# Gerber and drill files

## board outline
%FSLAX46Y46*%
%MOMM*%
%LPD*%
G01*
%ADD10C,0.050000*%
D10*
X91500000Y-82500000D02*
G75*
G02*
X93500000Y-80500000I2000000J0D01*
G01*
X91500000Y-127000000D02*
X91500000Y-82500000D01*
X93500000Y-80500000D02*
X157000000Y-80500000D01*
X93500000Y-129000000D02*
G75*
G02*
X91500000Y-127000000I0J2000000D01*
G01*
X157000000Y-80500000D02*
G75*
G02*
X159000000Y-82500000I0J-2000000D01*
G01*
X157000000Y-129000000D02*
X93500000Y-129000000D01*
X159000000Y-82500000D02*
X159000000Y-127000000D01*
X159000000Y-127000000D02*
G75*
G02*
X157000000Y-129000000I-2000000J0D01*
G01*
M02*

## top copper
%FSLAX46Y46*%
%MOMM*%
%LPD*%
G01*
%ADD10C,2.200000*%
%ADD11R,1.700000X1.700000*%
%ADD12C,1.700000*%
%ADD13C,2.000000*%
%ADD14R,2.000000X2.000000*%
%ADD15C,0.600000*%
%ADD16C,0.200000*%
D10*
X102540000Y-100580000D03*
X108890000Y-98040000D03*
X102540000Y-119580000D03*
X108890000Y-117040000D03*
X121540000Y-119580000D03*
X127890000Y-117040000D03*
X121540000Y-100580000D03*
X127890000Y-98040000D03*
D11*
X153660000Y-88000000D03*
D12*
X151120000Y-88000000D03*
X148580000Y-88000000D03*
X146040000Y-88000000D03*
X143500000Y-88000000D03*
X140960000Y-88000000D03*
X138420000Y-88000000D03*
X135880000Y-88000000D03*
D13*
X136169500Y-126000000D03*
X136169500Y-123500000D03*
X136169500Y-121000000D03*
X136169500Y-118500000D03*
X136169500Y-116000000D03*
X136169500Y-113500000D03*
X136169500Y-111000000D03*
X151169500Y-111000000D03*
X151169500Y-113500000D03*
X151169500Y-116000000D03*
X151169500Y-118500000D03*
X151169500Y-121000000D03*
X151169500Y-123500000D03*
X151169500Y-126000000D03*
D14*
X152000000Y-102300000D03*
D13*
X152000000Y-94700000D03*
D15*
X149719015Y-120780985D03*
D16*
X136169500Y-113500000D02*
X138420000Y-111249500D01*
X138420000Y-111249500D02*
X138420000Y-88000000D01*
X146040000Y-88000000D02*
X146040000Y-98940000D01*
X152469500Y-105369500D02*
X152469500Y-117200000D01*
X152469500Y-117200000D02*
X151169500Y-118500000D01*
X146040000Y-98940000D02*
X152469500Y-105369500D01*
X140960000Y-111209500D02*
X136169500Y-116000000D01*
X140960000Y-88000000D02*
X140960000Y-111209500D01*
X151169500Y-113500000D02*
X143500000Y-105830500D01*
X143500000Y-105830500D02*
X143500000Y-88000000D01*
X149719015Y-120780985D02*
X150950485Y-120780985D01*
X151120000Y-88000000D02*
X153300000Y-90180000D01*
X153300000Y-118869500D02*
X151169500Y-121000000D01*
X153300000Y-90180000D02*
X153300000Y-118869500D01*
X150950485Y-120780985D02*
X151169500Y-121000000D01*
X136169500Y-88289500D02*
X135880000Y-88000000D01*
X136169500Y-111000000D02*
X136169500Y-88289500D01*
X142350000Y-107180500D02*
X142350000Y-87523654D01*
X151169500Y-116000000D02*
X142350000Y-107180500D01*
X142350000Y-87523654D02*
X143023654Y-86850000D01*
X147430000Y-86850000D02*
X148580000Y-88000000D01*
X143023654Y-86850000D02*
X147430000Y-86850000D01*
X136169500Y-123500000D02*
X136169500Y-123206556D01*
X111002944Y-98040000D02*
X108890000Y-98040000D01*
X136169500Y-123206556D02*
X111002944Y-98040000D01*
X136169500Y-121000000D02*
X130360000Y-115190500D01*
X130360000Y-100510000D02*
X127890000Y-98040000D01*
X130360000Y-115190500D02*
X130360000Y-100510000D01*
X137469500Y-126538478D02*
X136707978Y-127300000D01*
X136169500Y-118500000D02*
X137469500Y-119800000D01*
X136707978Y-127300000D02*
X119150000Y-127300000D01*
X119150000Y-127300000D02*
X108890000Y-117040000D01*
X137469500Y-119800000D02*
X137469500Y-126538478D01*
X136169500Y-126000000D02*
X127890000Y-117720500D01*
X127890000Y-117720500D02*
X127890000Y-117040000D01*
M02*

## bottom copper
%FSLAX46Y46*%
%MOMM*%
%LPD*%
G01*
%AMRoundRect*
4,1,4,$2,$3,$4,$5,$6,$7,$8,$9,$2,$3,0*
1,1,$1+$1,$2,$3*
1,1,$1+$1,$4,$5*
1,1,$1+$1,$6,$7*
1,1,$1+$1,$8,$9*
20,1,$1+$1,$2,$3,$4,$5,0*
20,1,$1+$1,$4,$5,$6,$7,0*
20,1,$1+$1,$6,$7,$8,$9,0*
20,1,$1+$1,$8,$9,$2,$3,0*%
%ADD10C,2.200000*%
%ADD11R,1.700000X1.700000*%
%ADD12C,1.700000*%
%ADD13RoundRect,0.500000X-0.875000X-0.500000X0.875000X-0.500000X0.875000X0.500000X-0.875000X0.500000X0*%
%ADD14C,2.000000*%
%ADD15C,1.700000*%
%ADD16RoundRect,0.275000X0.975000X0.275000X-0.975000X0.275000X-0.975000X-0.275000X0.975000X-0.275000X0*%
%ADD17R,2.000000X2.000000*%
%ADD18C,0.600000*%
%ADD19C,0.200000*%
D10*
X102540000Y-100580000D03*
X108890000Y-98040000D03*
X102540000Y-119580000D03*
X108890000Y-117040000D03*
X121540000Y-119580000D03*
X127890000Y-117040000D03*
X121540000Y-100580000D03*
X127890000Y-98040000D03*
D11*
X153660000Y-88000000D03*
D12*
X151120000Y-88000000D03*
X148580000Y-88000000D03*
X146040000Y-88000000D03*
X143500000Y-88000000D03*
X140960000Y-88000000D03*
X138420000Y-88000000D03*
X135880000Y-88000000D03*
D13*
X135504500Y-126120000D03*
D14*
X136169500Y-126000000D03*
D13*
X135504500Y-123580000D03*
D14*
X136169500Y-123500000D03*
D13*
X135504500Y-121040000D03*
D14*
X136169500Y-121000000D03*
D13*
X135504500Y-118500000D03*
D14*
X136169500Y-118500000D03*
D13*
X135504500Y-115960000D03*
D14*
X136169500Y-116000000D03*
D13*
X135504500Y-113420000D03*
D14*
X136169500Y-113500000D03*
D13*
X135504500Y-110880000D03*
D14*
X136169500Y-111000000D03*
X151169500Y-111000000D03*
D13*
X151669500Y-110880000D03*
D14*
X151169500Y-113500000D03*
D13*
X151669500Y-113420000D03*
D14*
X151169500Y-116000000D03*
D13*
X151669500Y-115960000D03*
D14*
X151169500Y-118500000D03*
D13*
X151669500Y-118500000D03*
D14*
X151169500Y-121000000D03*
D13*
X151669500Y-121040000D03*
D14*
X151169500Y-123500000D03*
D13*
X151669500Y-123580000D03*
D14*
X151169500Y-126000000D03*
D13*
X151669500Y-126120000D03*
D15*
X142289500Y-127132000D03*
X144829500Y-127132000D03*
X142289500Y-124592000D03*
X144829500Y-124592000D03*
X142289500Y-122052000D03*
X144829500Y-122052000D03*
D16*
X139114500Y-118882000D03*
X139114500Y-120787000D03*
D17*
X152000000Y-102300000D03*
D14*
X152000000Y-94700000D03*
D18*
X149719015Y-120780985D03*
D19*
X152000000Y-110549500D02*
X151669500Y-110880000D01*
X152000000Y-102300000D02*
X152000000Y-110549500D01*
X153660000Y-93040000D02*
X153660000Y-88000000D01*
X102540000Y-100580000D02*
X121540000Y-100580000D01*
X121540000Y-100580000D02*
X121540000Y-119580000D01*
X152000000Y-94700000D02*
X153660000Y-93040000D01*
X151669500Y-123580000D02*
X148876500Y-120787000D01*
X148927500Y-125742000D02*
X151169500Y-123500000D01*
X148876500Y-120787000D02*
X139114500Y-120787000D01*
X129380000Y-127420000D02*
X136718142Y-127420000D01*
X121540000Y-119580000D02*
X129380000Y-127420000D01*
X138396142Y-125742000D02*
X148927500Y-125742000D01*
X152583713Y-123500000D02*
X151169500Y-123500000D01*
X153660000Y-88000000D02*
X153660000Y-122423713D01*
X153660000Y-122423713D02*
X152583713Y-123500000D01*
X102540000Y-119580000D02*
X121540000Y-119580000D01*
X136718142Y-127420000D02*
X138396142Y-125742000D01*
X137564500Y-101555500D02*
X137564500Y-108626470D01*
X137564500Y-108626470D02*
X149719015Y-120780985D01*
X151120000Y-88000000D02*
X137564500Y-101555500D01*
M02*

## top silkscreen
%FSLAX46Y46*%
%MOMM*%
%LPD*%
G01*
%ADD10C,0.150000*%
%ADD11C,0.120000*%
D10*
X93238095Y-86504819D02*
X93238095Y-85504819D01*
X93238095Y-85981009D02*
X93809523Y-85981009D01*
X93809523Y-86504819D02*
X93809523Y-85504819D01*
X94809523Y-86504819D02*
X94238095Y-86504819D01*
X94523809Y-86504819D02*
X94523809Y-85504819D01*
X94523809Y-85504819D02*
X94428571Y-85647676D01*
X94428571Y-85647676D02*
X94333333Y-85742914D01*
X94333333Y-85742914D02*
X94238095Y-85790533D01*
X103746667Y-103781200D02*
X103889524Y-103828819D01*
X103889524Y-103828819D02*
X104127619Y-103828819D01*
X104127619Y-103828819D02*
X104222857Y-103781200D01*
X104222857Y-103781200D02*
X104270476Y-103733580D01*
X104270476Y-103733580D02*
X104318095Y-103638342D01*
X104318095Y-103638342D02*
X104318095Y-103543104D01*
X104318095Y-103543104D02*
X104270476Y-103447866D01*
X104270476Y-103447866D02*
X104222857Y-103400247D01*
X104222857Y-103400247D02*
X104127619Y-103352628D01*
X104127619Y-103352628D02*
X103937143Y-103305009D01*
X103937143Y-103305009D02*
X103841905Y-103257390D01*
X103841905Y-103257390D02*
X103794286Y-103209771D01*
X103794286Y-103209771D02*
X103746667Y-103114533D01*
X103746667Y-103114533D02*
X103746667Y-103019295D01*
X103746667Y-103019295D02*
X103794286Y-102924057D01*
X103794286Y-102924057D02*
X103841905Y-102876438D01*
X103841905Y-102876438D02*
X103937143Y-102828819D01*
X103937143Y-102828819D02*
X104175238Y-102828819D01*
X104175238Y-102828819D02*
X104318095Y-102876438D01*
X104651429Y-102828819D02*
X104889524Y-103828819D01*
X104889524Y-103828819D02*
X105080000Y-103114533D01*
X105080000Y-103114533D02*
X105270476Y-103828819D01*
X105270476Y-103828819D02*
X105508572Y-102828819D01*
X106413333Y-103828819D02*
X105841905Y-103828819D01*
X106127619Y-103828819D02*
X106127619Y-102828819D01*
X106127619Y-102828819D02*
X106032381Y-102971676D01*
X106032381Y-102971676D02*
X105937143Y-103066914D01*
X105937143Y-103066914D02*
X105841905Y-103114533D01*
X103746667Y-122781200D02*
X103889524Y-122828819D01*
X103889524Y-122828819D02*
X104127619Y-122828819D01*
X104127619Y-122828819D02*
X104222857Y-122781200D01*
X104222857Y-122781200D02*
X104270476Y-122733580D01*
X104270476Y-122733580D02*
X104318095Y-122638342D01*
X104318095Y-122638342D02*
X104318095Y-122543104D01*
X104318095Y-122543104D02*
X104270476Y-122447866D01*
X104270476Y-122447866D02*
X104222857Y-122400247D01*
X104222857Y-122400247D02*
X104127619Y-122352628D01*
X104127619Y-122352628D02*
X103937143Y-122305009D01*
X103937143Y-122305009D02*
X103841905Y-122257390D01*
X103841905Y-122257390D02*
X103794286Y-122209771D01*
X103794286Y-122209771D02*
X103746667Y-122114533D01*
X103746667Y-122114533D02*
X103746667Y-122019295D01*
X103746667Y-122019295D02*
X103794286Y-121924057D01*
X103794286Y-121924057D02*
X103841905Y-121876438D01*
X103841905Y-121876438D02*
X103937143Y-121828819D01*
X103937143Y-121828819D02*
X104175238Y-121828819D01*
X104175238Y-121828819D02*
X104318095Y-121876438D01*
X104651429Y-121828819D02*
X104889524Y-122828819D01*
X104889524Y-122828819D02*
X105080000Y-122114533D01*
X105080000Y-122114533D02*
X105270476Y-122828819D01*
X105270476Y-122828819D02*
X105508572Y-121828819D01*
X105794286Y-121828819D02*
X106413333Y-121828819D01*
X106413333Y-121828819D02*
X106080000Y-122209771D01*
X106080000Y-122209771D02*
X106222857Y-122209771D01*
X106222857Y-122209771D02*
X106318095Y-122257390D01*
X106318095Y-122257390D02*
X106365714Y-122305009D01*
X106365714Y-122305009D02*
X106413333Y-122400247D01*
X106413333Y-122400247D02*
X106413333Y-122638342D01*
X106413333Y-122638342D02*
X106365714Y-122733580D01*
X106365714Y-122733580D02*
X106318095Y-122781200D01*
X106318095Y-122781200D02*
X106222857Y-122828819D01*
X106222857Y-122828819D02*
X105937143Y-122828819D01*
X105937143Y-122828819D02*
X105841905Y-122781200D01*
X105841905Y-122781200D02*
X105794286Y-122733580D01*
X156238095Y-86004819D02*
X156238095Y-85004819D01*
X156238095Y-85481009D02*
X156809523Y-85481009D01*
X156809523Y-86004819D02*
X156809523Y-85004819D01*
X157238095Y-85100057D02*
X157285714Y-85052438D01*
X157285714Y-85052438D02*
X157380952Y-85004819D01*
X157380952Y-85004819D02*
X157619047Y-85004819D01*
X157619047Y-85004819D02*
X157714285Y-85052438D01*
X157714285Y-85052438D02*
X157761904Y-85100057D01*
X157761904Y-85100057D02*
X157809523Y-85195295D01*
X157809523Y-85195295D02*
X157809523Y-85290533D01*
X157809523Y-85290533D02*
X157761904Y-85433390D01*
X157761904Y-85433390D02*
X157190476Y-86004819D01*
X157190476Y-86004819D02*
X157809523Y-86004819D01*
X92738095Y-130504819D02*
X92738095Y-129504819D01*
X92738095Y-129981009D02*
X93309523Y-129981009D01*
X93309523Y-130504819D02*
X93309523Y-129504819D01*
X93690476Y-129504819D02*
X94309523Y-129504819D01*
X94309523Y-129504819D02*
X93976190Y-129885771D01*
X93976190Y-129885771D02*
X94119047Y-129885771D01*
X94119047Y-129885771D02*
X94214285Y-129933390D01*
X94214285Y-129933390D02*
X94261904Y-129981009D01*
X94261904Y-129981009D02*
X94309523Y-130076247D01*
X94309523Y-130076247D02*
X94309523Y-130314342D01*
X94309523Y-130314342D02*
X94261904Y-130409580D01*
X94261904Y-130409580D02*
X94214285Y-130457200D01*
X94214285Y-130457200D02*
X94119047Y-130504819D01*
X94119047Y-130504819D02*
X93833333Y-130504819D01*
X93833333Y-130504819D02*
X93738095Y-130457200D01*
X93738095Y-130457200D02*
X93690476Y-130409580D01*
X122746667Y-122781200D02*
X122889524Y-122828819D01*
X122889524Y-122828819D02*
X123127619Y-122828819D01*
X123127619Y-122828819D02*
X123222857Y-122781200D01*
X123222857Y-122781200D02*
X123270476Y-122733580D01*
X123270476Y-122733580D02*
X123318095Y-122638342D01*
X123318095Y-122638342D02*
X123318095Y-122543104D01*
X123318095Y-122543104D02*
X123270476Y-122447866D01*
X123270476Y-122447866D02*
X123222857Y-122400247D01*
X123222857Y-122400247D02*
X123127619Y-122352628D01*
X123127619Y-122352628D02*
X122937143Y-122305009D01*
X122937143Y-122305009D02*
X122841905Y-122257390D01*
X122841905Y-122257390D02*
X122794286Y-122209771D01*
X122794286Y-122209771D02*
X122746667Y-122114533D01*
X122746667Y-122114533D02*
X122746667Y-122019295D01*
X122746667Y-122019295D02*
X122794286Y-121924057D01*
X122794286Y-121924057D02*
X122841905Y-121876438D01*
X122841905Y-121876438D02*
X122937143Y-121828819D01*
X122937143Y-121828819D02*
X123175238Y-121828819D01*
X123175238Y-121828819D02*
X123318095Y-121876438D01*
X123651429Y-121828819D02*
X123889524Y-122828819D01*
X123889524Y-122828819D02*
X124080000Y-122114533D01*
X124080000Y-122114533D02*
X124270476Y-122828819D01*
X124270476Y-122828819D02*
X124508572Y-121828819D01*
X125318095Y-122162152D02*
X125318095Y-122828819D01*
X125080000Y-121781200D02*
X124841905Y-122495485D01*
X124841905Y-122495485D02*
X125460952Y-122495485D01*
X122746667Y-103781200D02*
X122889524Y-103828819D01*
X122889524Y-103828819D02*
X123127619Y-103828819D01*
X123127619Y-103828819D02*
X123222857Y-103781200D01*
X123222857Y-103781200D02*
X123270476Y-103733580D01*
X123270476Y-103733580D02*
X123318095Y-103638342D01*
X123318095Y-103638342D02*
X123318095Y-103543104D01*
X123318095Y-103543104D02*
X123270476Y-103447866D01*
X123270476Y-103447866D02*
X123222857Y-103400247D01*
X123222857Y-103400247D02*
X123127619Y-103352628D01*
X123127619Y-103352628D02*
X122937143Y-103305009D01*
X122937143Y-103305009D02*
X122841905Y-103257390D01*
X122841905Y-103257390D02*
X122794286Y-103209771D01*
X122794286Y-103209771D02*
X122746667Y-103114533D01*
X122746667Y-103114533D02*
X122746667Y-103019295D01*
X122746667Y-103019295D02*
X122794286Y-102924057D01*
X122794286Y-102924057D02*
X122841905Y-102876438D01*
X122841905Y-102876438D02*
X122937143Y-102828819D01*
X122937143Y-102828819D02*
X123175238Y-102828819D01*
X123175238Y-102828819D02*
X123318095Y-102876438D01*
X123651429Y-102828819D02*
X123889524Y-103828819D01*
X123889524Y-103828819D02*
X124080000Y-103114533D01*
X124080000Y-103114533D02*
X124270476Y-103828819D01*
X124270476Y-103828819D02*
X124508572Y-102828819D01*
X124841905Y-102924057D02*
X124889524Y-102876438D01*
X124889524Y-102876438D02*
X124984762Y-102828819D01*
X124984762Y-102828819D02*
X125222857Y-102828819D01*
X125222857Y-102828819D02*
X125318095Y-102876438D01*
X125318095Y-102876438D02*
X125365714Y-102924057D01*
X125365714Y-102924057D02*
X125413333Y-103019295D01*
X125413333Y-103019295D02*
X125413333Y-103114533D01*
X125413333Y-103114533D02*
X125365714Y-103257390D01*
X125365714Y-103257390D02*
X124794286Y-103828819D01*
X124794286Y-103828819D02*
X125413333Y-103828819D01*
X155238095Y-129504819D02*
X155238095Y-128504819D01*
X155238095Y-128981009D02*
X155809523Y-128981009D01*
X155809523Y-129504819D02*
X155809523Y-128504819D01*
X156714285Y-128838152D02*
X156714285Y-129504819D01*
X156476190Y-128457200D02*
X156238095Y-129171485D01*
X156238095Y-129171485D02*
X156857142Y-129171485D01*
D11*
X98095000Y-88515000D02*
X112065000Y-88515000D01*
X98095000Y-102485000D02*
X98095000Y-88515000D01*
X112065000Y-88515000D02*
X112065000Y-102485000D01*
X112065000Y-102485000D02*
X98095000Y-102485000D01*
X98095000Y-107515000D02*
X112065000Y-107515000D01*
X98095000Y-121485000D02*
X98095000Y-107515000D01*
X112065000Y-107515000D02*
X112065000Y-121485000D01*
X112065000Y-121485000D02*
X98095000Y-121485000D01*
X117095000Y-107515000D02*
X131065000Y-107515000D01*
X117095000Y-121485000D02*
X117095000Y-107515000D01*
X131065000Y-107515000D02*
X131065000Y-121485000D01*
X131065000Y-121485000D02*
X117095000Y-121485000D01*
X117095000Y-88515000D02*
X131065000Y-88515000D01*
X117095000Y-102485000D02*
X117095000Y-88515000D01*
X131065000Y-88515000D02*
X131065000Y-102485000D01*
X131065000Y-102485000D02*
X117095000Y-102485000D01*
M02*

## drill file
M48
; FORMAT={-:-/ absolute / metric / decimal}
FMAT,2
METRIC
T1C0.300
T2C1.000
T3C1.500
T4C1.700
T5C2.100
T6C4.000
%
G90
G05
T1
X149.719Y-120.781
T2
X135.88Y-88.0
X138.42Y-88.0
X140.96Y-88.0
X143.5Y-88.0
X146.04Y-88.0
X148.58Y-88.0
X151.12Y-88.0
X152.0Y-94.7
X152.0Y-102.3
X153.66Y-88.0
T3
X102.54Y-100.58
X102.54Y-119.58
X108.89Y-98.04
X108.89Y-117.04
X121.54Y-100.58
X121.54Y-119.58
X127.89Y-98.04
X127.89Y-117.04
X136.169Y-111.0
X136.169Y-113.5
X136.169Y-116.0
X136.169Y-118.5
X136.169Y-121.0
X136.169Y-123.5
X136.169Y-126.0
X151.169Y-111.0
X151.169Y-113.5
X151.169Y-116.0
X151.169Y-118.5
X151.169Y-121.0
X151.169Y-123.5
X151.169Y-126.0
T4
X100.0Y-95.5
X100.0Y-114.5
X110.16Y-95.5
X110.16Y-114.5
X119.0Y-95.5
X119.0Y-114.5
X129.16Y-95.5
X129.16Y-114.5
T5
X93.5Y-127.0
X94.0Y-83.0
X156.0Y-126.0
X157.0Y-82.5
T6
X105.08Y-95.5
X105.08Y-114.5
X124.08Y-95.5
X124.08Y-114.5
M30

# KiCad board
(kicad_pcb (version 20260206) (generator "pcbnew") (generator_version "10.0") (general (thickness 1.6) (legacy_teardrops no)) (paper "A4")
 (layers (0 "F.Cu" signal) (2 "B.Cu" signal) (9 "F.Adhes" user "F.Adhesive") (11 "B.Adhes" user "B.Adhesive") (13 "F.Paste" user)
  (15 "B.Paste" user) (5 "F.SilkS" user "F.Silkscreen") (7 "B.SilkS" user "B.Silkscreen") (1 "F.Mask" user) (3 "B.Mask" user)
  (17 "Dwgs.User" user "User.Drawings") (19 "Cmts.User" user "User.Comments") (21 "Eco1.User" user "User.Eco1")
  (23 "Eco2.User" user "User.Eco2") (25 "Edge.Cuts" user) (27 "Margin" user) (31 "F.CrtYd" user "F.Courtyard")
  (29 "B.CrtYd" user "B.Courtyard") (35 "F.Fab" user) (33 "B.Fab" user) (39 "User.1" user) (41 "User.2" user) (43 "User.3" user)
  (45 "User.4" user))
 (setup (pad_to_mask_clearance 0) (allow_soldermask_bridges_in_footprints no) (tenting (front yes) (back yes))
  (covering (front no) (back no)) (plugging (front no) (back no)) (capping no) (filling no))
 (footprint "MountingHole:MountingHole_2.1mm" (layer "F.Cu") (at 94 83 180)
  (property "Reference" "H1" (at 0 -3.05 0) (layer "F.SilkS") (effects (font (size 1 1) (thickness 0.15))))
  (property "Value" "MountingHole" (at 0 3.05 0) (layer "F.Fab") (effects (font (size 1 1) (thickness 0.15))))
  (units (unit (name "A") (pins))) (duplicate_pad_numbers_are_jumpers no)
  (pad "" np_thru_hole circle (at 0 0 180) (size 2.1 2.1) (drill 2.1) (layers "*.Cu" "*.Mask")))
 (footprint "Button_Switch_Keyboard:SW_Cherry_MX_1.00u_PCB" (layer "F.Cu") (at 102.54 100.58 180)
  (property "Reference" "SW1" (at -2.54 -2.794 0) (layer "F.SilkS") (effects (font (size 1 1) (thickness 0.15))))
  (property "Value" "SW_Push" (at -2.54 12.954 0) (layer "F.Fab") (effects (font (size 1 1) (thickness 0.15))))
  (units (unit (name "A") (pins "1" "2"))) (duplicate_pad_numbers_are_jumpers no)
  (fp_line (start 4.445 12.065) (end -9.525 12.065) (stroke (width 0.12) (type solid)) (layer "F.SilkS"))
  (fp_line (start 4.445 -1.905) (end 4.445 12.065) (stroke (width 0.12) (type solid)) (layer "F.SilkS"))
  (fp_line (start -9.525 12.065) (end -9.525 -1.905) (stroke (width 0.12) (type solid)) (layer "F.SilkS"))
  (fp_line (start -9.525 -1.905) (end 4.445 -1.905) (stroke (width 0.12) (type solid)) (layer "F.SilkS"))
  (pad "" np_thru_hole circle (at -7.62 5.08 180) (size 1.7 1.7) (drill 1.7) (layers "*.Cu" "*.Mask"))
  (pad "" np_thru_hole circle (at -2.54 5.08 180) (size 4 4) (drill 4) (layers "*.Cu" "*.Mask"))
  (pad "" np_thru_hole circle (at 2.54 5.08 180) (size 1.7 1.7) (drill 1.7) (layers "*.Cu" "*.Mask"))
  (pad "1" thru_hole circle (at 0 0 180) (size 2.2 2.2) (drill 1.5) (layers "*.Cu" "*.Mask") (remove_unused_layers no) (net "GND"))
  (pad "2" thru_hole circle (at -6.35 2.54 180) (size 2.2 2.2) (drill 1.5) (layers "*.Cu" "*.Mask") (remove_unused_layers no)
   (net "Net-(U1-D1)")))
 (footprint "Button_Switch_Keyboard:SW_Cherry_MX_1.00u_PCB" (layer "F.Cu") (at 102.54 119.58 180)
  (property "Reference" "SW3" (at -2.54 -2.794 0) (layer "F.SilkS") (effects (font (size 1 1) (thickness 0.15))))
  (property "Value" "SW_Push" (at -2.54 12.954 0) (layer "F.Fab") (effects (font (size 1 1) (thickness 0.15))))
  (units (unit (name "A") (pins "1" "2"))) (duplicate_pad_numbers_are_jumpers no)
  (fp_line (start 4.445 12.065) (end -9.525 12.065) (stroke (width 0.12) (type solid)) (layer "F.SilkS"))
  (fp_line (start 4.445 -1.905) (end 4.445 12.065) (stroke (width 0.12) (type solid)) (layer "F.SilkS"))
  (fp_line (start -9.525 12.065) (end -9.525 -1.905) (stroke (width 0.12) (type solid)) (layer "F.SilkS"))
  (fp_line (start -9.525 -1.905) (end 4.445 -1.905) (stroke (width 0.12) (type solid)) (layer "F.SilkS"))
  (pad "" np_thru_hole circle (at -7.62 5.08 180) (size 1.7 1.7) (drill 1.7) (layers "*.Cu" "*.Mask"))
  (pad "" np_thru_hole circle (at -2.54 5.08 180) (size 4 4) (drill 4) (layers "*.Cu" "*.Mask"))
  (pad "" np_thru_hole circle (at 2.54 5.08 180) (size 1.7 1.7) (drill 1.7) (layers "*.Cu" "*.Mask"))
  (pad "1" thru_hole circle (at 0 0 180) (size 2.2 2.2) (drill 1.5) (layers "*.Cu" "*.Mask") (remove_unused_layers no) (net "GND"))
  (pad "2" thru_hole circle (at -6.35 2.54 180) (size 2.2 2.2) (drill 1.5) (layers "*.Cu" "*.Mask") (remove_unused_layers no)
   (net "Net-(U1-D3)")))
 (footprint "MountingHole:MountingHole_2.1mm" (layer "F.Cu") (at 157 82.5 180)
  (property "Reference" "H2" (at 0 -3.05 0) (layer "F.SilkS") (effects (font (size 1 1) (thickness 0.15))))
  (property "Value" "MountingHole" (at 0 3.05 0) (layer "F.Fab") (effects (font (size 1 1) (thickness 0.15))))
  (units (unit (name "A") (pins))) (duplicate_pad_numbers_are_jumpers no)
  (pad "" np_thru_hole circle (at 0 0 180) (size 2.1 2.1) (drill 2.1) (layers "*.Cu" "*.Mask")))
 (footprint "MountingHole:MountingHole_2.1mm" (layer "F.Cu") (at 93.5 127 180)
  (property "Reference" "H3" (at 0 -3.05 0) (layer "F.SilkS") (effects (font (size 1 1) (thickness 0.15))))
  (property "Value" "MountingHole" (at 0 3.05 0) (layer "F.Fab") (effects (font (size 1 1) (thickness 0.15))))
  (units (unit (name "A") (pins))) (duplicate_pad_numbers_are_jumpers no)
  (pad "" np_thru_hole circle (at 0 0 180) (size 2.1 2.1) (drill 2.1) (layers "*.Cu" "*.Mask")))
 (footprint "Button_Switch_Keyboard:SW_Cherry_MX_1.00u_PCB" (layer "F.Cu") (at 121.54 119.58 180)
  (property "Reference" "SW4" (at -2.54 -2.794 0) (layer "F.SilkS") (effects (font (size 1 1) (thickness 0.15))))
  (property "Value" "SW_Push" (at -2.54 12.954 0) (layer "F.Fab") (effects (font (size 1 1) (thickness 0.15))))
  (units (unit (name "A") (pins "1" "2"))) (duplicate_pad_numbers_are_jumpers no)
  (fp_line (start 4.445 12.065) (end -9.525 12.065) (stroke (width 0.12) (type solid)) (layer "F.SilkS"))
  (fp_line (start 4.445 -1.905) (end 4.445 12.065) (stroke (width 0.12) (type solid)) (layer "F.SilkS"))
  (fp_line (start -9.525 12.065) (end -9.525 -1.905) (stroke (width 0.12) (type solid)) (layer "F.SilkS"))
  (fp_line (start -9.525 -1.905) (end 4.445 -1.905) (stroke (width 0.12) (type solid)) (layer "F.SilkS"))
  (pad "" np_thru_hole circle (at -7.62 5.08 180) (size 1.7 1.7) (drill 1.7) (layers "*.Cu" "*.Mask"))
  (pad "" np_thru_hole circle (at -2.54 5.08 180) (size 4 4) (drill 4) (layers "*.Cu" "*.Mask"))
  (pad "" np_thru_hole circle (at 2.54 5.08 180) (size 1.7 1.7) (drill 1.7) (layers "*.Cu" "*.Mask"))
  (pad "1" thru_hole circle (at 0 0 180) (size 2.2 2.2) (drill 1.5) (layers "*.Cu" "*.Mask") (remove_unused_layers no) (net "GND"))
  (pad "2" thru_hole circle (at -6.35 2.54 180) (size 2.2 2.2) (drill 1.5) (layers "*.Cu" "*.Mask") (remove_unused_layers no)
   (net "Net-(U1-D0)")))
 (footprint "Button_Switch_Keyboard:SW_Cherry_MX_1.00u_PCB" (layer "F.Cu") (at 121.54 100.58 180)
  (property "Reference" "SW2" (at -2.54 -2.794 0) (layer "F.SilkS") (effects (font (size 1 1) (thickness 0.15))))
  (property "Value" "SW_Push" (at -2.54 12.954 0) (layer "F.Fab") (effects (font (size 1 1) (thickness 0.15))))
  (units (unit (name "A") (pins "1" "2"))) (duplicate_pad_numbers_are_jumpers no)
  (fp_line (start 4.445 12.065) (end -9.525 12.065) (stroke (width 0.12) (type solid)) (layer "F.SilkS"))
  (fp_line (start 4.445 -1.905) (end 4.445 12.065) (stroke (width 0.12) (type solid)) (layer "F.SilkS"))
  (fp_line (start -9.525 12.065) (end -9.525 -1.905) (stroke (width 0.12) (type solid)) (layer "F.SilkS"))
  (fp_line (start -9.525 -1.905) (end 4.445 -1.905) (stroke (width 0.12) (type solid)) (layer "F.SilkS"))
  (pad "" np_thru_hole circle (at -7.62 5.08 180) (size 1.7 1.7) (drill 1.7) (layers "*.Cu" "*.Mask"))
  (pad "" np_thru_hole circle (at -2.54 5.08 180) (size 4 4) (drill 4) (layers "*.Cu" "*.Mask"))
  (pad "" np_thru_hole circle (at 2.54 5.08 180) (size 1.7 1.7) (drill 1.7) (layers "*.Cu" "*.Mask"))
  (pad "1" thru_hole circle (at 0 0 180) (size 2.2 2.2) (drill 1.5) (layers "*.Cu" "*.Mask") (remove_unused_layers no) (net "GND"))
  (pad "2" thru_hole circle (at -6.35 2.54 180) (size 2.2 2.2) (drill 1.5) (layers "*.Cu" "*.Mask") (remove_unused_layers no)
   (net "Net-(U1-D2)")))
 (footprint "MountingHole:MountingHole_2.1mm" (layer "F.Cu") (at 156 126 180)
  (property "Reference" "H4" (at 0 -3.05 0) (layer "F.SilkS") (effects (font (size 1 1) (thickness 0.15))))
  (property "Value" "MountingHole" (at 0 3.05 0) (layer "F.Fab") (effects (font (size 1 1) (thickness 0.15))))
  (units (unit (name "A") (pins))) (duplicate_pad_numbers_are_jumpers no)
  (pad "" np_thru_hole circle (at 0 0 180) (size 2.1 2.1) (drill 2.1) (layers "*.Cu" "*.Mask")))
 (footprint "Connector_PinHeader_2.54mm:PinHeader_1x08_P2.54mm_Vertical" (layer "B.Cu") (at 153.66 88 90)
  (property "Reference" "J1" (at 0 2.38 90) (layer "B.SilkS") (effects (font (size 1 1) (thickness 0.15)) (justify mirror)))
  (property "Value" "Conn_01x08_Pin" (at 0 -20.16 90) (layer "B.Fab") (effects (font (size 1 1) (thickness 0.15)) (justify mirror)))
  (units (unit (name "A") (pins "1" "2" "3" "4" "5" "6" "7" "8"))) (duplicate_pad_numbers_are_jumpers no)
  (pad "1" thru_hole rect (at 0 0 90) (size 1.7 1.7) (drill 1) (layers "*.Cu" "*.Mask") (remove_unused_layers no) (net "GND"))
  (pad "2" thru_hole circle (at 0 -2.54 90) (size 1.7 1.7) (drill 1) (layers "*.Cu" "*.Mask") (remove_unused_layers no) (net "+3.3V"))
  (pad "3" thru_hole circle (at 0 -5.08 90) (size 1.7 1.7) (drill 1) (layers "*.Cu" "*.Mask") (remove_unused_layers no) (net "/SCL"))
  (pad "4" thru_hole circle (at 0 -7.62 90) (size 1.7 1.7) (drill 1) (layers "*.Cu" "*.Mask") (remove_unused_layers no) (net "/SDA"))
  (pad "5" thru_hole circle (at 0 -10.16 90) (size 1.7 1.7) (drill 1) (layers "*.Cu" "*.Mask") (remove_unused_layers no) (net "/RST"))
  (pad "6" thru_hole circle (at 0 -12.7 90) (size 1.7 1.7) (drill 1) (layers "*.Cu" "*.Mask") (remove_unused_layers no) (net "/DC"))
  (pad "7" thru_hole circle (at 0 -15.24 90) (size 1.7 1.7) (drill 1) (layers "*.Cu" "*.Mask") (remove_unused_layers no) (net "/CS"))
  (pad "8" thru_hole circle (at 0 -17.78 90) (size 1.7 1.7) (drill 1) (layers "*.Cu" "*.Mask") (remove_unused_layers no) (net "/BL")))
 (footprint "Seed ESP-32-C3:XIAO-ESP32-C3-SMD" (layer "B.Cu") (at 134.6695 108)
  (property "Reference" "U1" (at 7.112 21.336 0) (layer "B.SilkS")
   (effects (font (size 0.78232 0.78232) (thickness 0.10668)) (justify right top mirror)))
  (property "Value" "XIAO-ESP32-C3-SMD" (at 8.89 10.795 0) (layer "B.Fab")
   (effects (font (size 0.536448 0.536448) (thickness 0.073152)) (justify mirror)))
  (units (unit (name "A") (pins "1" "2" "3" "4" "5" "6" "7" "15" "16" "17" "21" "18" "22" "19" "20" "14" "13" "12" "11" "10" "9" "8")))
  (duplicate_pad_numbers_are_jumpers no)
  (pad "1" smd roundrect (at 0.835 18.12) (size 2.75 2) (layers "B.Cu" "B.Mask" "B.Paste") (roundrect_rratio 0.25) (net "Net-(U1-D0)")
   (solder_mask_margin 0.0508) (thermal_bridge_angle 45))
  (pad "1" thru_hole circle (at 1.5 18) (size 2 2) (drill 1.5) (layers "*.Cu" "*.Mask") (remove_unused_layers no) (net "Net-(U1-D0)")
   (thermal_bridge_angle 90))
  (pad "2" smd roundrect (at 0.835 15.58) (size 2.75 2) (layers "B.Cu" "B.Mask" "B.Paste") (roundrect_rratio 0.25) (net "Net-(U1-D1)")
   (solder_mask_margin 0.0508) (thermal_bridge_angle 45))
  (pad "2" thru_hole circle (at 1.5 15.5) (size 2 2) (drill 1.5) (layers "*.Cu" "*.Mask") (remove_unused_layers no) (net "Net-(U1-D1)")
   (thermal_bridge_angle 90))
  (pad "3" smd roundrect (at 0.835 13.04) (size 2.75 2) (layers "B.Cu" "B.Mask" "B.Paste") (roundrect_rratio 0.25) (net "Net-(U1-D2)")
   (solder_mask_margin 0.0508) (thermal_bridge_angle 45))
  (pad "3" thru_hole circle (at 1.5 13) (size 2 2) (drill 1.5) (layers "*.Cu" "*.Mask") (remove_unused_layers no) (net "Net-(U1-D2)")
   (thermal_bridge_angle 90))
  (pad "4" smd roundrect (at 0.835 10.5) (size 2.75 2) (layers "B.Cu" "B.Mask" "B.Paste") (roundrect_rratio 0.25) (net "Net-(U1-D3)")
   (solder_mask_margin 0.0508) (thermal_bridge_angle 45))
  (pad "4" thru_hole circle (at 1.5 10.5) (size 2 2) (drill 1.5) (layers "*.Cu" "*.Mask") (remove_unused_layers no) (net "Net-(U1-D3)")
   (thermal_bridge_angle 90))
  (pad "5" smd roundrect (at 0.835 7.96) (size 2.75 2) (layers "B.Cu" "B.Mask" "B.Paste") (roundrect_rratio 0.25) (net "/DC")
   (solder_mask_margin 0.0508) (thermal_bridge_angle 45))
  (pad "5" thru_hole circle (at 1.5 8) (size 2 2) (drill 1.5) (layers "*.Cu" "*.Mask") (remove_unused_layers no) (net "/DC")
   (thermal_bridge_angle 90))
  (pad "6" smd roundrect (at 0.835 5.42) (size 2.75 2) (layers "B.Cu" "B.Mask" "B.Paste") (roundrect_rratio 0.25) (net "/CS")
   (solder_mask_margin 0.0508) (thermal_bridge_angle 45))
  (pad "6" thru_hole circle (at 1.5 5.5) (size 2 2) (drill 1.5) (layers "*.Cu" "*.Mask") (remove_unused_layers no) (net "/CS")
   (thermal_bridge_angle 90))
  (pad "7" smd roundrect (at 0.835 2.88) (size 2.75 2) (layers "B.Cu" "B.Mask" "B.Paste") (roundrect_rratio 0.25) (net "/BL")
   (solder_mask_margin 0.0508) (thermal_bridge_angle 45))
  (pad "7" thru_hole circle (at 1.5 3) (size 2 2) (drill 1.5) (layers "*.Cu" "*.Mask") (remove_unused_layers no) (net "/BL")
   (thermal_bridge_angle 90))
  (pad "8" thru_hole circle (at 16.5 3) (size 2 2) (drill 1.5) (layers "*.Cu" "*.Mask") (remove_unused_layers no) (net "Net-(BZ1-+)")
   (thermal_bridge_angle 90))
  (pad "8" smd roundrect (at 17 2.88) (size 2.75 2) (layers "B.Cu" "B.Mask" "B.Paste") (roundrect_rratio 0.25) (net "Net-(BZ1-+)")
   (solder_mask_margin 0.0508) (thermal_bridge_angle 45))
  (pad "9" thru_hole circle (at 16.5 5.5) (size 2 2) (drill 1.5) (layers "*.Cu" "*.Mask") (remove_unused_layers no) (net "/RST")
   (thermal_bridge_angle 90))
  (pad "9" smd roundrect (at 17 5.42) (size 2.75 2) (layers "B.Cu" "B.Mask" "B.Paste") (roundrect_rratio 0.25) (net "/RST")
   (solder_mask_margin 0.0508) (thermal_bridge_angle 45))
  (pad "10" thru_hole circle (at 16.5 8) (size 2 2) (drill 1.5) (layers "*.Cu" "*.Mask") (remove_unused_layers no) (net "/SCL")
   (thermal_bridge_angle 90))
  (pad "10" smd roundrect (at 17 7.96) (size 2.75 2) (layers "B.Cu" "B.Mask" "B.Paste") (roundrect_rratio 0.25) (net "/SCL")
   (solder_mask_margin 0.0508) (thermal_bridge_angle 45))
  (pad "11" thru_hole circle (at 16.5 10.5) (size 2 2) (drill 1.5) (layers "*.Cu" "*.Mask") (remove_unused_layers no) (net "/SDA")
   (thermal_bridge_angle 90))
  (pad "11" smd roundrect (at 17 10.5) (size 2.75 2) (layers "B.Cu" "B.Mask" "B.Paste") (roundrect_rratio 0.25) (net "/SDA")
   (solder_mask_margin 0.0508) (thermal_bridge_angle 45))
  (pad "12" thru_hole circle (at 16.5 13) (size 2 2) (drill 1.5) (layers "*.Cu" "*.Mask") (remove_unused_layers no) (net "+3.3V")
   (thermal_bridge_angle 90))
  (pad "12" smd roundrect (at 17 13.04) (size 2.75 2) (layers "B.Cu" "B.Mask" "B.Paste") (roundrect_rratio 0.25) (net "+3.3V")
   (solder_mask_margin 0.0508) (thermal_bridge_angle 45))
  (pad "13" thru_hole circle (at 16.5 15.5) (size 2 2) (drill 1.5) (layers "*.Cu" "*.Mask") (remove_unused_layers no) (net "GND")
   (thermal_bridge_angle 90))
  (pad "13" smd roundrect (at 17 15.58) (size 2.75 2) (layers "B.Cu" "B.Mask" "B.Paste") (roundrect_rratio 0.25) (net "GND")
   (solder_mask_margin 0.0508) (thermal_bridge_angle 45))
  (pad "14" thru_hole circle (at 16.5 18) (size 2 2) (drill 1.5) (layers "*.Cu" "*.Mask") (remove_unused_layers no)
   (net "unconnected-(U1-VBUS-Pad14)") (thermal_bridge_angle 90))
  (pad "14" smd roundrect (at 17 18.12) (size 2.75 2) (layers "B.Cu" "B.Mask" "B.Paste") (roundrect_rratio 0.25)
   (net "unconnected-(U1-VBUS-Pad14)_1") (solder_mask_margin 0.0508) (thermal_bridge_angle 45))
  (pad "15" smd circle (at 7.62 19.132) (size 1.7 1.7) (layers "B.Cu" "B.Mask" "B.Paste") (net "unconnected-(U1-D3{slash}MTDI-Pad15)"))
  (pad "16" smd circle (at 10.16 19.132) (size 1.7 1.7) (layers "B.Cu" "B.Mask" "B.Paste") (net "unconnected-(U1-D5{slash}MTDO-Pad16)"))
  (pad "17" smd circle (at 7.62 16.592) (size 1.7 1.7) (layers "B.Cu" "B.Mask" "B.Paste") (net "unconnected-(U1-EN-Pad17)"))
  (pad "18" smd circle (at 10.16 16.592) (size 1.7 1.7) (layers "B.Cu" "B.Mask" "B.Paste") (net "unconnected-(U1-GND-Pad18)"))
  (pad "19" smd circle (at 7.62 14.052) (size 1.7 1.7) (layers "B.Cu" "B.Mask" "B.Paste") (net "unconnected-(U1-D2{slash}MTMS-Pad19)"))
  (pad "20" smd circle (at 10.16 14.052) (size 1.7 1.7) (layers "B.Cu" "B.Mask" "B.Paste") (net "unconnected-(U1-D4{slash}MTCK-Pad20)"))
  (pad "21" smd roundrect (at 4.445 10.882 180) (size 2.5 1.1) (layers "B.Cu" "B.Mask" "B.Paste") (roundrect_rratio 0.25)
   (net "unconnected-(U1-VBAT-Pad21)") (thermal_bridge_angle 45))
  (pad "22" smd roundrect (at 4.445 12.787 180) (size 2.5 1.1) (layers "B.Cu" "B.Mask" "B.Paste") (roundrect_rratio 0.25) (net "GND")
   (thermal_bridge_angle 45)))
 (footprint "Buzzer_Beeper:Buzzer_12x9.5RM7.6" (layer "B.Cu") (at 152 102.3 90)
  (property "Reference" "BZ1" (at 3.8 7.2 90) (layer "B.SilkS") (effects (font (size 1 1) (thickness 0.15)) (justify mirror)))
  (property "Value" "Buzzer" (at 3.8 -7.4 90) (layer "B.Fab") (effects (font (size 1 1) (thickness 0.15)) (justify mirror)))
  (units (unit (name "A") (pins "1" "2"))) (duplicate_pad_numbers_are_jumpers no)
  (pad "1" thru_hole rect (at 0 0 90) (size 2 2) (drill 1) (layers "*.Cu" "*.Mask") (remove_unused_layers no) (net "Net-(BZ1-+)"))
  (pad "2" thru_hole circle (at 7.6 0 90) (size 2 2) (drill 1) (layers "*.Cu" "*.Mask") (remove_unused_layers no) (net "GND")))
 (gr_arc (start 91.5 82.5) (mid 92.085786 81.085786) (end 93.5 80.5) (stroke (width 0.05) (type default)) (layer "Edge.Cuts"))
 (gr_line (start 91.5 127) (end 91.5 82.5) (stroke (width 0.05) (type default)) (layer "Edge.Cuts"))
 (gr_line (start 93.5 80.5) (end 157 80.5) (stroke (width 0.05) (type default)) (layer "Edge.Cuts"))
 (gr_arc (start 93.5 129) (mid 92.085786 128.414214) (end 91.5 127) (stroke (width 0.05) (type default)) (layer "Edge.Cuts"))
 (gr_arc (start 157 80.5) (mid 158.414214 81.085786) (end 159 82.5) (stroke (width 0.05) (type default)) (layer "Edge.Cuts"))
 (gr_line (start 157 129) (end 93.5 129) (stroke (width 0.05) (type default)) (layer "Edge.Cuts"))
 (gr_line (start 159 82.5) (end 159 127) (stroke (width 0.05) (type default)) (layer "Edge.Cuts"))
 (gr_arc (start 159 127) (mid 158.414214 128.414214) (end 157 129) (stroke (width 0.05) (type default)) (layer "Edge.Cuts"))
 (segment (start 152 110.5495) (end 151.6695 110.88) (width 0.2) (layer "B.Cu") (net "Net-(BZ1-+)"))
 (segment (start 152 102.3) (end 152 110.5495) (width 0.2) (layer "B.Cu") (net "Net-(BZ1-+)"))
 (segment (start 153.66 93.04) (end 153.66 88) (width 0.2) (layer "B.Cu") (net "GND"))
 (segment (start 102.54 100.58) (end 121.54 100.58) (width 0.2) (layer "B.Cu") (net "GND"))
 (segment (start 121.54 100.58) (end 121.54 119.58) (width 0.2) (layer "B.Cu") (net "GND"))
 (segment (start 152 94.7) (end 153.66 93.04) (width 0.2) (layer "B.Cu") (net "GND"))
 (segment (start 151.6695 123.58) (end 148.8765 120.787) (width 0.2) (layer "B.Cu") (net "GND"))
 (segment (start 148.9275 125.742) (end 151.1695 123.5) (width 0.2) (layer "B.Cu") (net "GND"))
 (segment (start 148.8765 120.787) (end 139.1145 120.787) (width 0.2) (layer "B.Cu") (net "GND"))
 (segment (start 129.38 127.42) (end 136.718142 127.42) (width 0.2) (layer "B.Cu") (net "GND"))
 (segment (start 121.54 119.58) (end 129.38 127.42) (width 0.2) (layer "B.Cu") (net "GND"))
 (segment (start 138.396142 125.742) (end 148.9275 125.742) (width 0.2) (layer "B.Cu") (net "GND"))
 (segment (start 152.583713 123.5) (end 151.1695 123.5) (width 0.2) (layer "B.Cu") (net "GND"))
 (segment (start 153.66 88) (end 153.66 122.423713) (width 0.2) (layer "B.Cu") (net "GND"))
 (segment (start 153.66 122.423713) (end 152.583713 123.5) (width 0.2) (layer "B.Cu") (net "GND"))
 (segment (start 102.54 119.58) (end 121.54 119.58) (width 0.2) (layer "B.Cu") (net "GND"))
 (segment (start 136.718142 127.42) (end 138.396142 125.742) (width 0.2) (layer "B.Cu") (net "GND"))
 (segment (start 136.1695 113.5) (end 138.42 111.2495) (width 0.2) (layer "F.Cu") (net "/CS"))
 (segment (start 138.42 111.2495) (end 138.42 88) (width 0.2) (layer "F.Cu") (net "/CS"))
 (segment (start 146.04 88) (end 146.04 98.94) (width 0.2) (layer "F.Cu") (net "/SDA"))
 (segment (start 152.4695 105.3695) (end 152.4695 117.2) (width 0.2) (layer "F.Cu") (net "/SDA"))
 (segment (start 152.4695 117.2) (end 151.1695 118.5) (width 0.2) (layer "F.Cu") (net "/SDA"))
 (segment (start 146.04 98.94) (end 152.4695 105.3695) (width 0.2) (layer "F.Cu") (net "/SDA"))
 (segment (start 140.96 111.2095) (end 136.1695 116) (width 0.2) (layer "F.Cu") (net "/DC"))
 (segment (start 140.96 88) (end 140.96 111.2095) (width 0.2) (layer "F.Cu") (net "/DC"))
 (segment (start 151.1695 113.5) (end 143.5 105.8305) (width 0.2) (layer "F.Cu") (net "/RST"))
 (segment (start 143.5 105.8305) (end 143.5 88) (width 0.2) (layer "F.Cu") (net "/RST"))
 (segment (start 149.719015 120.780985) (end 150.950485 120.780985) (width 0.2) (layer "F.Cu") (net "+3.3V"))
 (segment (start 151.12 88) (end 153.3 90.18) (width 0.2) (layer "F.Cu") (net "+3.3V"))
 (segment (start 153.3 118.8695) (end 151.1695 121) (width 0.2) (layer "F.Cu") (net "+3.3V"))
 (segment (start 153.3 90.18) (end 153.3 118.8695) (width 0.2) (layer "F.Cu") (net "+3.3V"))
 (segment (start 150.950485 120.780985) (end 151.1695 121) (width 0.2) (layer "F.Cu") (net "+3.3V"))
 (via (at 149.719015 120.780985) (size 0.6) (drill 0.3) (layers "F.Cu" "B.Cu") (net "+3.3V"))
 (segment (start 137.5645 101.5555) (end 137.5645 108.62647) (width 0.2) (layer "B.Cu") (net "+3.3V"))
 (segment (start 137.5645 108.62647) (end 149.719015 120.780985) (width 0.2) (layer "B.Cu") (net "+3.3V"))
 (segment (start 151.12 88) (end 137.5645 101.5555) (width 0.2) (layer "B.Cu") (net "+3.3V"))
 (segment (start 136.1695 88.2895) (end 135.88 88) (width 0.2) (layer "F.Cu") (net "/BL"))
 (segment (start 136.1695 111) (end 136.1695 88.2895) (width 0.2) (layer "F.Cu") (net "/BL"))
 (segment (start 142.35 107.1805) (end 142.35 87.523654) (width 0.2) (layer "F.Cu") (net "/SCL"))
 (segment (start 151.1695 116) (end 142.35 107.1805) (width 0.2) (layer "F.Cu") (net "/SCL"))
 (segment (start 142.35 87.523654) (end 143.023654 86.85) (width 0.2) (layer "F.Cu") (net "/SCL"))
 (segment (start 147.43 86.85) (end 148.58 88) (width 0.2) (layer "F.Cu") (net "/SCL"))
 (segment (start 143.023654 86.85) (end 147.43 86.85) (width 0.2) (layer "F.Cu") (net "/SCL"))
 (segment (start 136.1695 123.5) (end 136.1695 123.206556) (width 0.2) (layer "F.Cu") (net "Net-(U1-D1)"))
 (segment (start 111.002944 98.04) (end 108.89 98.04) (width 0.2) (layer "F.Cu") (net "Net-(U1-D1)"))
 (segment (start 136.1695 123.206556) (end 111.002944 98.04) (width 0.2) (layer "F.Cu") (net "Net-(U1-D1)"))
 (segment (start 136.1695 121) (end 130.36 115.1905) (width 0.2) (layer "F.Cu") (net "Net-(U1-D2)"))
 (segment (start 130.36 100.51) (end 127.89 98.04) (width 0.2) (layer "F.Cu") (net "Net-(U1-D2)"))
 (segment (start 130.36 115.1905) (end 130.36 100.51) (width 0.2) (layer "F.Cu") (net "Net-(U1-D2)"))
 (segment (start 137.4695 126.538478) (end 136.707978 127.3) (width 0.2) (layer "F.Cu") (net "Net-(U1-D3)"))
 (segment (start 136.1695 118.5) (end 137.4695 119.8) (width 0.2) (layer "F.Cu") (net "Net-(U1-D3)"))
 (segment (start 136.707978 127.3) (end 119.15 127.3) (width 0.2) (layer "F.Cu") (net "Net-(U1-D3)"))
 (segment (start 119.15 127.3) (end 108.89 117.04) (width 0.2) (layer "F.Cu") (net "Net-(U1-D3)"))
 (segment (start 137.4695 119.8) (end 137.4695 126.538478) (width 0.2) (layer "F.Cu") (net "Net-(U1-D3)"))
 (segment (start 136.1695 126) (end 127.89 117.7205) (width 0.2) (layer "F.Cu") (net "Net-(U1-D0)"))
 (segment (start 127.89 117.7205) (end 127.89 117.04) (width 0.2) (layer "F.Cu") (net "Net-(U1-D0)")))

